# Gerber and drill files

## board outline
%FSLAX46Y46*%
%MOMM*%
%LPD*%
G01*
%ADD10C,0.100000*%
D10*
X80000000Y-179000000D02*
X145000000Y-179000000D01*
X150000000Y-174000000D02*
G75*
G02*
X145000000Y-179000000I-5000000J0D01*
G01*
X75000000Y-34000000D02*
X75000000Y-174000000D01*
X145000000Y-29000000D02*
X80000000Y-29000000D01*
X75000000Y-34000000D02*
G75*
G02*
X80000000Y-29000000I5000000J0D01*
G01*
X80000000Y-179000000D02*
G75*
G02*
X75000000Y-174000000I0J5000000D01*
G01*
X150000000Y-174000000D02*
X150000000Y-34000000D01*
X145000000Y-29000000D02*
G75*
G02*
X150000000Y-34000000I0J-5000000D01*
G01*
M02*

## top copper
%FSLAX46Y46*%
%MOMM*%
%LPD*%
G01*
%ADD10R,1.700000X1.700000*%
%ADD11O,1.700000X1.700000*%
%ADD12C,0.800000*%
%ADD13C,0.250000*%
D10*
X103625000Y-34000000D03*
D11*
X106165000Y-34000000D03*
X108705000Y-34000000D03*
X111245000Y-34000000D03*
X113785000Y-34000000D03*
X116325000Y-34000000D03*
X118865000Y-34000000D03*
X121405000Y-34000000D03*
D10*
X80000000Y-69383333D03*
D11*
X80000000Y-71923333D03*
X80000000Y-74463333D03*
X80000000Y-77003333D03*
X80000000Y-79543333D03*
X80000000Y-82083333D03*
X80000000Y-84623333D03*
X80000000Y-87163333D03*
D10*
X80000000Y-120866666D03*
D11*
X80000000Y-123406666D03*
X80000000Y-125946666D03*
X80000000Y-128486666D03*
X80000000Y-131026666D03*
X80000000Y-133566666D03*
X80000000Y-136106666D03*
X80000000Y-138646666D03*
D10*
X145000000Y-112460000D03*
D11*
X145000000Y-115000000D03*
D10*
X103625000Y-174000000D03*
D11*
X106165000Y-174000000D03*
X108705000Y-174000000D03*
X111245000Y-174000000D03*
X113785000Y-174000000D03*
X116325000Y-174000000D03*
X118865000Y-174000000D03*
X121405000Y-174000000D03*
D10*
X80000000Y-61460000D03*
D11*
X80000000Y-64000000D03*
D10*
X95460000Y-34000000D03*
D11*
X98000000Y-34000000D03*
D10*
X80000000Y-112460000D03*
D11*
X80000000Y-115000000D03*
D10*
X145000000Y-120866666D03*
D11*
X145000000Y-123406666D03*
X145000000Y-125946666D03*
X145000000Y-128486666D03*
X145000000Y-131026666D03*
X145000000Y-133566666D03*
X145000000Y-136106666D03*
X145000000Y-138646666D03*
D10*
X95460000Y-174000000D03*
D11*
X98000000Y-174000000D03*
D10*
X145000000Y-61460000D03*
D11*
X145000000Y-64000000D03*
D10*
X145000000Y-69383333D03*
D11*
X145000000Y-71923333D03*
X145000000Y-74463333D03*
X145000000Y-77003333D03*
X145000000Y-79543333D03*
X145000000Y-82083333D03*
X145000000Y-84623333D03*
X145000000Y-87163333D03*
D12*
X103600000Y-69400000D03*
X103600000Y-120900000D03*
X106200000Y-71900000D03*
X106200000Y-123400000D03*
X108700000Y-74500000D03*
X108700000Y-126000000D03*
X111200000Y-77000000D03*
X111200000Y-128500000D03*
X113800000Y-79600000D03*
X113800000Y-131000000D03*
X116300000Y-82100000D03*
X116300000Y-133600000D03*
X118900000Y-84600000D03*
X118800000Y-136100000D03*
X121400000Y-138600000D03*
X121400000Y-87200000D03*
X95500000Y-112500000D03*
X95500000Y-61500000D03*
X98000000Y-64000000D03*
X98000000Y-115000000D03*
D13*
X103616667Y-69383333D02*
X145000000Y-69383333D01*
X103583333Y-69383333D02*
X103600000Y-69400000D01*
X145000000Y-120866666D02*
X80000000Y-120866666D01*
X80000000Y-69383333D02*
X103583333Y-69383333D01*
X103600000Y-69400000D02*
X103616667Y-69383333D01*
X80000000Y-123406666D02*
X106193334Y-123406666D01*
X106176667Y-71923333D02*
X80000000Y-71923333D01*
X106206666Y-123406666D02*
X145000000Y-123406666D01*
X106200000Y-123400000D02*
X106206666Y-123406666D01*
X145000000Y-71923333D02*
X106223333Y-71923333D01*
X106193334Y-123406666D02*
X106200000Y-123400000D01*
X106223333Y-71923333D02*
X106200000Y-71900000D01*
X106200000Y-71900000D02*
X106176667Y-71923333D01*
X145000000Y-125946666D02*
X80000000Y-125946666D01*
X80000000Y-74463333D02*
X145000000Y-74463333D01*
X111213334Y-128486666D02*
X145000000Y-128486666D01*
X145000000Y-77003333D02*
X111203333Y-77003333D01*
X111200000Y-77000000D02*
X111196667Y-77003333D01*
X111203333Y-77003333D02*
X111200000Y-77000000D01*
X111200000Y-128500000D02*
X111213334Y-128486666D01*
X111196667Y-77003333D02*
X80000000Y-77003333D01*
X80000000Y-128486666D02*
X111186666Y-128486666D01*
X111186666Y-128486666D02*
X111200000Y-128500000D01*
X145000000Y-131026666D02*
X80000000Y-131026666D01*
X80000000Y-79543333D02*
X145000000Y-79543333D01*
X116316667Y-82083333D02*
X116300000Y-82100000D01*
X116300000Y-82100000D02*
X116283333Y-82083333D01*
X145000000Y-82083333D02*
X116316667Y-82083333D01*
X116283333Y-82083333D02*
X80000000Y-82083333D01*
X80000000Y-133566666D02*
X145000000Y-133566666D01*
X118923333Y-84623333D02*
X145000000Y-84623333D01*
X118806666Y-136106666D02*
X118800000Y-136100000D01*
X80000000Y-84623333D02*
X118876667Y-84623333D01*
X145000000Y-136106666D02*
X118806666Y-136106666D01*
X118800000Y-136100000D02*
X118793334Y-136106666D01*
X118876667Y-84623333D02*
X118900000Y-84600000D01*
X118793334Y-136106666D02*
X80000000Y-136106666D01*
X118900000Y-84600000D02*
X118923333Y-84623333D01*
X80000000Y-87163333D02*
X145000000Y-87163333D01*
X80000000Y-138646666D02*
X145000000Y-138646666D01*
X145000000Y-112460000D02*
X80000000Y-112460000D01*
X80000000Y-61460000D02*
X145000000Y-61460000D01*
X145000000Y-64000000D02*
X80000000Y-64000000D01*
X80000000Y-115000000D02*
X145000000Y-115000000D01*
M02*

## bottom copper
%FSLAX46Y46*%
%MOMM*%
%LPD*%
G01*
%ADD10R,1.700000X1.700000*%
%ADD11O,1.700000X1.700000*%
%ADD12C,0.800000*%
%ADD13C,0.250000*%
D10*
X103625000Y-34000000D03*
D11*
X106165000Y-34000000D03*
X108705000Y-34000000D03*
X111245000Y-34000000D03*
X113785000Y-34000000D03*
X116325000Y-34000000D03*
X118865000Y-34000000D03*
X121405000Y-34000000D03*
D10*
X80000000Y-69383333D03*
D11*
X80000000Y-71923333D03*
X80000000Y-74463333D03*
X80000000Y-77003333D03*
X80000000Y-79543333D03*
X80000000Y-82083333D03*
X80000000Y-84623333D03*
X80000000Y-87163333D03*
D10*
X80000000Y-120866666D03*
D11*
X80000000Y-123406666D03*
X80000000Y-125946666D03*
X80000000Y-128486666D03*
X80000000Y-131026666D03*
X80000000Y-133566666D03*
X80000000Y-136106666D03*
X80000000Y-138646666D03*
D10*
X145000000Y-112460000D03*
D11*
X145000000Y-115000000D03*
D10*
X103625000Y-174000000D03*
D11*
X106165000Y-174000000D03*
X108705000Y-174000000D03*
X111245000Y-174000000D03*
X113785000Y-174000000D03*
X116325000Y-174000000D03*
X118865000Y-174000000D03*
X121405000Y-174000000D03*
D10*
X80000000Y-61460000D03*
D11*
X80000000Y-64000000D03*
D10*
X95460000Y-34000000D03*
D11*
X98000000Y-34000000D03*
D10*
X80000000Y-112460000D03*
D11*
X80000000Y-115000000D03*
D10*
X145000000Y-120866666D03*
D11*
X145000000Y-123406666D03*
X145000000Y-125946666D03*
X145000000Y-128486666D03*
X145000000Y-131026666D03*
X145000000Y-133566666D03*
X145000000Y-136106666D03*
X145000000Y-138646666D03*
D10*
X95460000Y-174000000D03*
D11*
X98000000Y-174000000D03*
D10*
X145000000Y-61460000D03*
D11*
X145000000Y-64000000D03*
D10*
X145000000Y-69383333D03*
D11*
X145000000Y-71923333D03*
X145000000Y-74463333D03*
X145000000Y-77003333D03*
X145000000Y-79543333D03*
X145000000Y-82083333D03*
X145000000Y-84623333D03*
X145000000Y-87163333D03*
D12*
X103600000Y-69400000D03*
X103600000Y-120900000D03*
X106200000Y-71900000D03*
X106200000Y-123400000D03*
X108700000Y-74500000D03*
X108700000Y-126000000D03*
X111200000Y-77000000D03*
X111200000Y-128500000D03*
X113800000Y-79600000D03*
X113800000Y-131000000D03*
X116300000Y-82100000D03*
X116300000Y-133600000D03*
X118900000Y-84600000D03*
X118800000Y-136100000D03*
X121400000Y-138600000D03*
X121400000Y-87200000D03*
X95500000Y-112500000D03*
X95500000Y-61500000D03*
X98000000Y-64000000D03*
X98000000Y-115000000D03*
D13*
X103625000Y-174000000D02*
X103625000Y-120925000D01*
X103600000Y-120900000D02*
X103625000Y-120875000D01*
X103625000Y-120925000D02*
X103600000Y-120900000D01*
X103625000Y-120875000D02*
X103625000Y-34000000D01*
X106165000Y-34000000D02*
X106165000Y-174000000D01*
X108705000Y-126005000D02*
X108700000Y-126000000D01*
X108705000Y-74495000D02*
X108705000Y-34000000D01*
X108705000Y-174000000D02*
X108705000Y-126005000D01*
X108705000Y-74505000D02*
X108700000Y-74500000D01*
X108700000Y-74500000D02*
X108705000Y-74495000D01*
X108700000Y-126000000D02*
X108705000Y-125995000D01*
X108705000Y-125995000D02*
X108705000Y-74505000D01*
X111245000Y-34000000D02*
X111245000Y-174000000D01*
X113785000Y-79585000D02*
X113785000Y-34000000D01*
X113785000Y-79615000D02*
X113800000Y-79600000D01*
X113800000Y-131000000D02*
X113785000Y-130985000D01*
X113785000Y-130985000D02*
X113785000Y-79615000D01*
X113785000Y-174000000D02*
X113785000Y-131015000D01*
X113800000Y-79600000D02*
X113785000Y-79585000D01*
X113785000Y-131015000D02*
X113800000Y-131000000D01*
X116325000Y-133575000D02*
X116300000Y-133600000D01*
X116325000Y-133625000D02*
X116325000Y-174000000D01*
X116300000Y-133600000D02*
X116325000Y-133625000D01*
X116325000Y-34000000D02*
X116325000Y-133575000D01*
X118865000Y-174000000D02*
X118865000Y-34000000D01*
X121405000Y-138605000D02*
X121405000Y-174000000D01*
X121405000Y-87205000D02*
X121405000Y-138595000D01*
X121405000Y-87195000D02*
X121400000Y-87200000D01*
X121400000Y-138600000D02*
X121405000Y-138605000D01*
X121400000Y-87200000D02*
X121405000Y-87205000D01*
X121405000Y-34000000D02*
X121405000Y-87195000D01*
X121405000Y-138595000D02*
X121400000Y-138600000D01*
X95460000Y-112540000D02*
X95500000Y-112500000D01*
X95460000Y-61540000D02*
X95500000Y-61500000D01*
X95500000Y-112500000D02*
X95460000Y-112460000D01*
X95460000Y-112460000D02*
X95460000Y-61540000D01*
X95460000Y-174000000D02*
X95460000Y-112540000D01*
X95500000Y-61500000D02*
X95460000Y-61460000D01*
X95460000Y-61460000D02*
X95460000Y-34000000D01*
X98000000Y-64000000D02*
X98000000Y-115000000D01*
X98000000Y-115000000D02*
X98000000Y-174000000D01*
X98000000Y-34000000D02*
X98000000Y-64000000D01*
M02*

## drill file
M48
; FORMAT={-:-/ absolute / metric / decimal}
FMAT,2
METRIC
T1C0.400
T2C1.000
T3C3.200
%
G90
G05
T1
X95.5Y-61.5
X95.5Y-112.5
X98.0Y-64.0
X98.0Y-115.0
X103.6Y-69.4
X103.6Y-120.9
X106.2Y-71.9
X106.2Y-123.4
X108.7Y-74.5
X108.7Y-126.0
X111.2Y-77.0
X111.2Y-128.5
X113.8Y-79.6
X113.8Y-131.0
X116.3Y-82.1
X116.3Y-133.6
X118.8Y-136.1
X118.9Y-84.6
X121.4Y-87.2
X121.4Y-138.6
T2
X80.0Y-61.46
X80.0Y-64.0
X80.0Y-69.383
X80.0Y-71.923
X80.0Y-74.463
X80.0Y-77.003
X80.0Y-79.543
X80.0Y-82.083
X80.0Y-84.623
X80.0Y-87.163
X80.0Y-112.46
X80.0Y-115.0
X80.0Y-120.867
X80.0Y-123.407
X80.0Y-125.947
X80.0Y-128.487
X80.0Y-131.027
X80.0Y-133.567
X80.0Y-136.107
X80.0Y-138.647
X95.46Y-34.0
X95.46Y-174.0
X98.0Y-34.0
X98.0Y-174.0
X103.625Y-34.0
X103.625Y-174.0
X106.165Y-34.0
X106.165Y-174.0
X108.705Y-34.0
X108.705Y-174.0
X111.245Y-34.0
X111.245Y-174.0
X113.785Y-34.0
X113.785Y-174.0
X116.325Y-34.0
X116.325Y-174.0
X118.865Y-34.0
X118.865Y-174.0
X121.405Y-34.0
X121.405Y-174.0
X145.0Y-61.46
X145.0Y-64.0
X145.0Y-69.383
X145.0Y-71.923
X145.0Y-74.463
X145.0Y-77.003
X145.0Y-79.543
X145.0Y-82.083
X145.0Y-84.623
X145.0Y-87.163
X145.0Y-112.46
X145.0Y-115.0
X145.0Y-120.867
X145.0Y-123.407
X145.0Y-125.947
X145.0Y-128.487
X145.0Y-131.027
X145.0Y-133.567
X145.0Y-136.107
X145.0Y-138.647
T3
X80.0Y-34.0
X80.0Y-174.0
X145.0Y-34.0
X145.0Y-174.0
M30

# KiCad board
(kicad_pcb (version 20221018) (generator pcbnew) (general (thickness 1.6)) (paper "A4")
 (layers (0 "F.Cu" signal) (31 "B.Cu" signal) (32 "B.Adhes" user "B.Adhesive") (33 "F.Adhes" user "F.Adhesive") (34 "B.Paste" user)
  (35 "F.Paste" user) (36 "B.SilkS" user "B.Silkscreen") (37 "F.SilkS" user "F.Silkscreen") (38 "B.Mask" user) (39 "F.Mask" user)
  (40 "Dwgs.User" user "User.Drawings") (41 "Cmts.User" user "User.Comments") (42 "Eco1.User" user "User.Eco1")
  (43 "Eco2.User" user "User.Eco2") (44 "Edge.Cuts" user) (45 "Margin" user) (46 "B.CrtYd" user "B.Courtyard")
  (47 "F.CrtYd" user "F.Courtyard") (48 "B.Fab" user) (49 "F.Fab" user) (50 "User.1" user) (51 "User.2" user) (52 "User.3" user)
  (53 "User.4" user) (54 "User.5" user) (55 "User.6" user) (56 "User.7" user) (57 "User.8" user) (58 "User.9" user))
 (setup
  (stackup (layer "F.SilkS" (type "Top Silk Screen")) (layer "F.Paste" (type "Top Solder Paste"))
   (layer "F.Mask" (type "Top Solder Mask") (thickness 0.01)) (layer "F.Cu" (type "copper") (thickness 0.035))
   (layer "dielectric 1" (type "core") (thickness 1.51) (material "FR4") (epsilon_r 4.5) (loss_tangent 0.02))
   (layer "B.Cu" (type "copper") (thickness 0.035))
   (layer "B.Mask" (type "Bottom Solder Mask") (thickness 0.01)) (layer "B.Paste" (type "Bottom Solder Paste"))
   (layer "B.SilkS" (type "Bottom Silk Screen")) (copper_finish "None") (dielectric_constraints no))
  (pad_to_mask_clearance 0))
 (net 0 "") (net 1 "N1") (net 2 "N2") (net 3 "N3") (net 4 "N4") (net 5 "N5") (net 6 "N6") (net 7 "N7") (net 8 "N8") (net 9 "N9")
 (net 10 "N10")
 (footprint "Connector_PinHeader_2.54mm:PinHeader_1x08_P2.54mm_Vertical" (layer "F.Cu") (at 103.625 34 90)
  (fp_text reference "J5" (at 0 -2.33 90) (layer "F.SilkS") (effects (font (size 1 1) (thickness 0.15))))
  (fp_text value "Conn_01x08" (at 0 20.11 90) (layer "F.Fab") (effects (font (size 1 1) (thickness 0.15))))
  (pad "1" thru_hole rect (at 0 0 90) (size 1.7 1.7) (drill 1) (layers "*.Cu" "*.Mask") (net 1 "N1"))
  (pad "2" thru_hole oval (at 0 2.54 90) (size 1.7 1.7) (drill 1) (layers "*.Cu" "*.Mask") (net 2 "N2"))
  (pad "3" thru_hole oval (at 0 5.08 90) (size 1.7 1.7) (drill 1) (layers "*.Cu" "*.Mask") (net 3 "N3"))
  (pad "4" thru_hole oval (at 0 7.62 90) (size 1.7 1.7) (drill 1) (layers "*.Cu" "*.Mask") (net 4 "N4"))
  (pad "5" thru_hole oval (at 0 10.16 90) (size 1.7 1.7) (drill 1) (layers "*.Cu" "*.Mask") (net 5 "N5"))
  (pad "6" thru_hole oval (at 0 12.7 90) (size 1.7 1.7) (drill 1) (layers "*.Cu" "*.Mask") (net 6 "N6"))
  (pad "7" thru_hole oval (at 0 15.24 90) (size 1.7 1.7) (drill 1) (layers "*.Cu" "*.Mask") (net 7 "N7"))
  (pad "8" thru_hole oval (at 0 17.78 90) (size 1.7 1.7) (drill 1) (layers "*.Cu" "*.Mask") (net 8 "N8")))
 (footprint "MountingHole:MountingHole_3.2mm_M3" (layer "F.Cu") (at 80 174)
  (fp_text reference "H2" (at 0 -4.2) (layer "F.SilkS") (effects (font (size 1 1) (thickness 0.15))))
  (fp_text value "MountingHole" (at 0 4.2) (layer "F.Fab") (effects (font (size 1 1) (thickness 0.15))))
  (pad "" np_thru_hole circle (at 0 0) (size 3.2 3.2) (drill 3.2) (layers "*.Cu" "*.Mask")))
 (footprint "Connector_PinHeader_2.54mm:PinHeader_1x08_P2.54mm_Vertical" (layer "F.Cu") (at 80 69.383333)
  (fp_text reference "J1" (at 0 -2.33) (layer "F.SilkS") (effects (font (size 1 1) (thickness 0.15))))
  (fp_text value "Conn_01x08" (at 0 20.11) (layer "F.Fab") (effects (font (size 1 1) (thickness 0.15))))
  (pad "1" thru_hole rect (at 0 0) (size 1.7 1.7) (drill 1) (layers "*.Cu" "*.Mask") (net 1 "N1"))
  (pad "2" thru_hole oval (at 0 2.54) (size 1.7 1.7) (drill 1) (layers "*.Cu" "*.Mask") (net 2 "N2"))
  (pad "3" thru_hole oval (at 0 5.08) (size 1.7 1.7) (drill 1) (layers "*.Cu" "*.Mask") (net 3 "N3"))
  (pad "4" thru_hole oval (at 0 7.62) (size 1.7 1.7) (drill 1) (layers "*.Cu" "*.Mask") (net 4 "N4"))
  (pad "5" thru_hole oval (at 0 10.16) (size 1.7 1.7) (drill 1) (layers "*.Cu" "*.Mask") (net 5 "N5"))
  (pad "6" thru_hole oval (at 0 12.7) (size 1.7 1.7) (drill 1) (layers "*.Cu" "*.Mask") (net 6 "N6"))
  (pad "7" thru_hole oval (at 0 15.24) (size 1.7 1.7) (drill 1) (layers "*.Cu" "*.Mask") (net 7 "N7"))
  (pad "8" thru_hole oval (at 0 17.78) (size 1.7 1.7) (drill 1) (layers "*.Cu" "*.Mask") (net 8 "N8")))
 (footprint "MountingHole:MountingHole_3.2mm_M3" (layer "F.Cu") (at 145 174)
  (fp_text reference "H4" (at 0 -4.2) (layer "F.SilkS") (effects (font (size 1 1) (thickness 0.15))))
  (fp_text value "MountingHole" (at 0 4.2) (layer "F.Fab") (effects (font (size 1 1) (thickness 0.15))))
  (pad "" np_thru_hole circle (at 0 0) (size 3.2 3.2) (drill 3.2) (layers "*.Cu" "*.Mask")))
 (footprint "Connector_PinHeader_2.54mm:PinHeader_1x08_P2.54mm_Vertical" (layer "F.Cu") (at 80 120.866666)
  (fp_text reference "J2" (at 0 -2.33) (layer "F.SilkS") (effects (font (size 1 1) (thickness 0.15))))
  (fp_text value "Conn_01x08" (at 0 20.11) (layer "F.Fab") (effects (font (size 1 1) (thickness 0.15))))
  (pad "1" thru_hole rect (at 0 0) (size 1.7 1.7) (drill 1) (layers "*.Cu" "*.Mask") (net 1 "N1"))
  (pad "2" thru_hole oval (at 0 2.54) (size 1.7 1.7) (drill 1) (layers "*.Cu" "*.Mask") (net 2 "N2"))
  (pad "3" thru_hole oval (at 0 5.08) (size 1.7 1.7) (drill 1) (layers "*.Cu" "*.Mask") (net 3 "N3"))
  (pad "4" thru_hole oval (at 0 7.62) (size 1.7 1.7) (drill 1) (layers "*.Cu" "*.Mask") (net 4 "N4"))
  (pad "5" thru_hole oval (at 0 10.16) (size 1.7 1.7) (drill 1) (layers "*.Cu" "*.Mask") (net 5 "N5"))
  (pad "6" thru_hole oval (at 0 12.7) (size 1.7 1.7) (drill 1) (layers "*.Cu" "*.Mask") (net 6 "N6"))
  (pad "7" thru_hole oval (at 0 15.24) (size 1.7 1.7) (drill 1) (layers "*.Cu" "*.Mask") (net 7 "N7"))
  (pad "8" thru_hole oval (at 0 17.78) (size 1.7 1.7) (drill 1) (layers "*.Cu" "*.Mask") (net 8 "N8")))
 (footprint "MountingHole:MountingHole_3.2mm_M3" (layer "F.Cu") (at 80 34)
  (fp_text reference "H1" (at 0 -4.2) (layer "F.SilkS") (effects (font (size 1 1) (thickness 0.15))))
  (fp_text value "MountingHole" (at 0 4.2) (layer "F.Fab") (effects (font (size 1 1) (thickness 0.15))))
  (pad "" np_thru_hole circle (at 0 0) (size 3.2 3.2) (drill 3.2) (layers "*.Cu" "*.Mask")))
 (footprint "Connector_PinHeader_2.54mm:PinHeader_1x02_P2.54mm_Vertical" (layer "F.Cu") (at 145 112.46)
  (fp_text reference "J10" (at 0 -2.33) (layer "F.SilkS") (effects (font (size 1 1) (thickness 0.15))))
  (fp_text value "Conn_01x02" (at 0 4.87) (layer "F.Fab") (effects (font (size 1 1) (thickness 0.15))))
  (pad "1" thru_hole rect (at 0 0) (size 1.7 1.7) (drill 1) (layers "*.Cu" "*.Mask") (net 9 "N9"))
  (pad "2" thru_hole oval (at 0 2.54) (size 1.7 1.7) (drill 1) (layers "*.Cu" "*.Mask") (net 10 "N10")))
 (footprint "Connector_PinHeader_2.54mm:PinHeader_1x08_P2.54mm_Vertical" (layer "F.Cu") (at 103.625 174 90)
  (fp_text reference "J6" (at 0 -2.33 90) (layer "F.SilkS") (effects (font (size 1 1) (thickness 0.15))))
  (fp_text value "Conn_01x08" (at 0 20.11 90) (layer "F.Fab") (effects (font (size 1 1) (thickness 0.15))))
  (pad "1" thru_hole rect (at 0 0 90) (size 1.7 1.7) (drill 1) (layers "*.Cu" "*.Mask") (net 1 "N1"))
  (pad "2" thru_hole oval (at 0 2.54 90) (size 1.7 1.7) (drill 1) (layers "*.Cu" "*.Mask") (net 2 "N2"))
  (pad "3" thru_hole oval (at 0 5.08 90) (size 1.7 1.7) (drill 1) (layers "*.Cu" "*.Mask") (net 3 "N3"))
  (pad "4" thru_hole oval (at 0 7.62 90) (size 1.7 1.7) (drill 1) (layers "*.Cu" "*.Mask") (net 4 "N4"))
  (pad "5" thru_hole oval (at 0 10.16 90) (size 1.7 1.7) (drill 1) (layers "*.Cu" "*.Mask") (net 5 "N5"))
  (pad "6" thru_hole oval (at 0 12.7 90) (size 1.7 1.7) (drill 1) (layers "*.Cu" "*.Mask") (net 6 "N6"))
  (pad "7" thru_hole oval (at 0 15.24 90) (size 1.7 1.7) (drill 1) (layers "*.Cu" "*.Mask") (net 7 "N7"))
  (pad "8" thru_hole oval (at 0 17.78 90) (size 1.7 1.7) (drill 1) (layers "*.Cu" "*.Mask") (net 8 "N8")))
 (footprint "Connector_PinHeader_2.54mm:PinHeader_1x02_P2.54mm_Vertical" (layer "F.Cu") (at 80 61.46)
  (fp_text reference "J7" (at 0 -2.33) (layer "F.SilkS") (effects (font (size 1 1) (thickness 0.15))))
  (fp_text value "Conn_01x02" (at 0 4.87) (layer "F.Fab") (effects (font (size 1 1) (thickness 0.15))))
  (pad "1" thru_hole rect (at 0 0) (size 1.7 1.7) (drill 1) (layers "*.Cu" "*.Mask") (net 9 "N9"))
  (pad "2" thru_hole oval (at 0 2.54) (size 1.7 1.7) (drill 1) (layers "*.Cu" "*.Mask") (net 10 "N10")))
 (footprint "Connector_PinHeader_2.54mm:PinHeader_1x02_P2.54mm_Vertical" (layer "F.Cu") (at 95.46 34 90)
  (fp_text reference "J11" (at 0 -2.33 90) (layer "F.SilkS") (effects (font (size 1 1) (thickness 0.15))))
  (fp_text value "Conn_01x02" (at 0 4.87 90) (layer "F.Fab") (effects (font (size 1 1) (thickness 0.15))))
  (pad "1" thru_hole rect (at 0 0 90) (size 1.7 1.7) (drill 1) (layers "*.Cu" "*.Mask") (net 9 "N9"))
  (pad "2" thru_hole oval (at 0 2.54 90) (size 1.7 1.7) (drill 1) (layers "*.Cu" "*.Mask") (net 10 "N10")))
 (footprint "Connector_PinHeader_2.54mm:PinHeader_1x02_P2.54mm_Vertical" (layer "F.Cu") (at 80 112.46)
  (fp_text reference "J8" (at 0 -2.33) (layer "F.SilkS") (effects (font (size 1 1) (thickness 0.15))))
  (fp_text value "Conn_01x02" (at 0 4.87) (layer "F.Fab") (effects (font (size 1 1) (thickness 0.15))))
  (pad "1" thru_hole rect (at 0 0) (size 1.7 1.7) (drill 1) (layers "*.Cu" "*.Mask") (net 9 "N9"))
  (pad "2" thru_hole oval (at 0 2.54) (size 1.7 1.7) (drill 1) (layers "*.Cu" "*.Mask") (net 10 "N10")))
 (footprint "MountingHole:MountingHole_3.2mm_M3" (layer "F.Cu") (at 145 34)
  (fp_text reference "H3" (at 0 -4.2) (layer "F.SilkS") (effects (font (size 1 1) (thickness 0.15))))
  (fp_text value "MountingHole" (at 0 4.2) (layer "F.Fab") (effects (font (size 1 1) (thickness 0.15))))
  (pad "" np_thru_hole circle (at 0 0) (size 3.2 3.2) (drill 3.2) (layers "*.Cu" "*.Mask")))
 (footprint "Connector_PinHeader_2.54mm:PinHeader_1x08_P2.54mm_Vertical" (layer "F.Cu") (at 145 120.866666)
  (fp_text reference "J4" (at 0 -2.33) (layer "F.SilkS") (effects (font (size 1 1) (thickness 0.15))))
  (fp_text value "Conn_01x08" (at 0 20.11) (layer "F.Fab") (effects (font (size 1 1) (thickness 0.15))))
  (pad "1" thru_hole rect (at 0 0) (size 1.7 1.7) (drill 1) (layers "*.Cu" "*.Mask") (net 1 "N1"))
  (pad "2" thru_hole oval (at 0 2.54) (size 1.7 1.7) (drill 1) (layers "*.Cu" "*.Mask") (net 2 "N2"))
  (pad "3" thru_hole oval (at 0 5.08) (size 1.7 1.7) (drill 1) (layers "*.Cu" "*.Mask") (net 3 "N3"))
  (pad "4" thru_hole oval (at 0 7.62) (size 1.7 1.7) (drill 1) (layers "*.Cu" "*.Mask") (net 4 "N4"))
  (pad "5" thru_hole oval (at 0 10.16) (size 1.7 1.7) (drill 1) (layers "*.Cu" "*.Mask") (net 5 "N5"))
  (pad "6" thru_hole oval (at 0 12.7) (size 1.7 1.7) (drill 1) (layers "*.Cu" "*.Mask") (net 6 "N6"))
  (pad "7" thru_hole oval (at 0 15.24) (size 1.7 1.7) (drill 1) (layers "*.Cu" "*.Mask") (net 7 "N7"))
  (pad "8" thru_hole oval (at 0 17.78) (size 1.7 1.7) (drill 1) (layers "*.Cu" "*.Mask") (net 8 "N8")))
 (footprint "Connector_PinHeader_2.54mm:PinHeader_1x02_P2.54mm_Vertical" (layer "F.Cu") (at 95.46 174 90)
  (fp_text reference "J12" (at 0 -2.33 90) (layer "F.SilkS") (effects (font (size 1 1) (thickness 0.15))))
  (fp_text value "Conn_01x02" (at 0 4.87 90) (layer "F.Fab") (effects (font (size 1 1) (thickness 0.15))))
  (pad "1" thru_hole rect (at 0 0 90) (size 1.7 1.7) (drill 1) (layers "*.Cu" "*.Mask") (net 9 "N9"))
  (pad "2" thru_hole oval (at 0 2.54 90) (size 1.7 1.7) (drill 1) (layers "*.Cu" "*.Mask") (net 10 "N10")))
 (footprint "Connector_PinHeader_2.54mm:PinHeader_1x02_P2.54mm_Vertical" (layer "F.Cu") (at 145 61.46)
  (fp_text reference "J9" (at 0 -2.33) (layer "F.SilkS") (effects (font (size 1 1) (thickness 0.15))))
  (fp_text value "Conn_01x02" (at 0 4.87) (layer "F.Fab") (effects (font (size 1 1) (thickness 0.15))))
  (pad "1" thru_hole rect (at 0 0) (size 1.7 1.7) (drill 1) (layers "*.Cu" "*.Mask") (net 9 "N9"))
  (pad "2" thru_hole oval (at 0 2.54) (size 1.7 1.7) (drill 1) (layers "*.Cu" "*.Mask") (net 10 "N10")))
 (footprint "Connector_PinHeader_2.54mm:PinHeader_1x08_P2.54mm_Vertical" (layer "F.Cu") (at 145 69.383333)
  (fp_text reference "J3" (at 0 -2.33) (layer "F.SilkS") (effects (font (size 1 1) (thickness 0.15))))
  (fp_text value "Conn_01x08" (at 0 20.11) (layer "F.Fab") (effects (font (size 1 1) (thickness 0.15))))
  (pad "1" thru_hole rect (at 0 0) (size 1.7 1.7) (drill 1) (layers "*.Cu" "*.Mask") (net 1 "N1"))
  (pad "2" thru_hole oval (at 0 2.54) (size 1.7 1.7) (drill 1) (layers "*.Cu" "*.Mask") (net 2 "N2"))
  (pad "3" thru_hole oval (at 0 5.08) (size 1.7 1.7) (drill 1) (layers "*.Cu" "*.Mask") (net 3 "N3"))
  (pad "4" thru_hole oval (at 0 7.62) (size 1.7 1.7) (drill 1) (layers "*.Cu" "*.Mask") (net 4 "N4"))
  (pad "5" thru_hole oval (at 0 10.16) (size 1.7 1.7) (drill 1) (layers "*.Cu" "*.Mask") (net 5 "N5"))
  (pad "6" thru_hole oval (at 0 12.7) (size 1.7 1.7) (drill 1) (layers "*.Cu" "*.Mask") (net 6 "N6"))
  (pad "7" thru_hole oval (at 0 15.24) (size 1.7 1.7) (drill 1) (layers "*.Cu" "*.Mask") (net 7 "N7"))
  (pad "8" thru_hole oval (at 0 17.78) (size 1.7 1.7) (drill 1) (layers "*.Cu" "*.Mask") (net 8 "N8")))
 (gr_line (start 80 179) (end 145 179) (stroke (width 0.1) (type default)) (layer "Edge.Cuts"))
 (gr_arc (start 150 174) (mid 148.535534 177.535534) (end 145 179) (stroke (width 0.1) (type default)) (layer "Edge.Cuts"))
 (gr_line (start 75 34) (end 75 174) (stroke (width 0.1) (type default)) (layer "Edge.Cuts"))
 (gr_line (start 145 29) (end 80 29) (stroke (width 0.1) (type default)) (layer "Edge.Cuts"))
 (gr_arc (start 75 34) (mid 76.464466 30.464466) (end 80 29) (stroke (width 0.1) (type default)) (layer "Edge.Cuts"))
 (gr_arc (start 80 179) (mid 76.464466 177.535534) (end 75 174) (stroke (width 0.1) (type default)) (layer "Edge.Cuts"))
 (gr_line (start 150 174) (end 150 34) (stroke (width 0.1) (type default)) (layer "Edge.Cuts"))
 (gr_arc (start 145 29) (mid 148.535534 30.464466) (end 150 34) (stroke (width 0.1) (type default)) (layer "Edge.Cuts"))
 (segment (start 103.616667 69.383333) (end 145 69.383333) (width 0.25) (layer "F.Cu") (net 1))
 (segment (start 103.583333 69.383333) (end 103.6 69.4) (width 0.25) (layer "F.Cu") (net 1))
 (segment (start 145 120.866666) (end 80 120.866666) (width 0.25) (layer "F.Cu") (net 1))
 (segment (start 80 69.383333) (end 103.583333 69.383333) (width 0.25) (layer "F.Cu") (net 1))
 (segment (start 103.6 69.4) (end 103.616667 69.383333) (width 0.25) (layer "F.Cu") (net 1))
 (via (at 103.6 69.4) (size 0.8) (drill 0.4) (layers "F.Cu" "B.Cu") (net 1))
 (via (at 103.6 120.9) (size 0.8) (drill 0.4) (layers "F.Cu" "B.Cu") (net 1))
 (segment (start 103.625 174) (end 103.625 120.925) (width 0.25) (layer "B.Cu") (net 1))
 (segment (start 103.6 120.9) (end 103.625 120.875) (width 0.25) (layer "B.Cu") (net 1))
 (segment (start 103.625 120.925) (end 103.6 120.9) (width 0.25) (layer "B.Cu") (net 1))
 (segment (start 103.625 120.875) (end 103.625 34) (width 0.25) (layer "B.Cu") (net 1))
 (segment (start 80 123.406666) (end 106.193334 123.406666) (width 0.25) (layer "F.Cu") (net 2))
 (segment (start 106.176667 71.923333) (end 80 71.923333) (width 0.25) (layer "F.Cu") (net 2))
 (segment (start 106.206666 123.406666) (end 145 123.406666) (width 0.25) (layer "F.Cu") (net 2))
 (segment (start 106.2 123.4) (end 106.206666 123.406666) (width 0.25) (layer "F.Cu") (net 2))
 (segment (start 145 71.923333) (end 106.223333 71.923333) (width 0.25) (layer "F.Cu") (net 2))
 (segment (start 106.193334 123.406666) (end 106.2 123.4) (width 0.25) (layer "F.Cu") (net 2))
 (segment (start 106.223333 71.923333) (end 106.2 71.9) (width 0.25) (layer "F.Cu") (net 2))
 (segment (start 106.2 71.9) (end 106.176667 71.923333) (width 0.25) (layer "F.Cu") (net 2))
 (via (at 106.2 71.9) (size 0.8) (drill 0.4) (layers "F.Cu" "B.Cu") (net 2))
 (via (at 106.2 123.4) (size 0.8) (drill 0.4) (layers "F.Cu" "B.Cu") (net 2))
 (segment (start 106.165 34) (end 106.165 174) (width 0.25) (layer "B.Cu") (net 2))
 (segment (start 145 125.946666) (end 80 125.946666) (width 0.25) (layer "F.Cu") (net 3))
 (segment (start 80 74.463333) (end 145 74.463333) (width 0.25) (layer "F.Cu") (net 3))
 (via (at 108.7 74.5) (size 0.8) (drill 0.4) (layers "F.Cu" "B.Cu") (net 3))
 (via (at 108.7 126) (size 0.8) (drill 0.4) (layers "F.Cu" "B.Cu") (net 3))
 (segment (start 108.705 126.005) (end 108.7 126) (width 0.25) (layer "B.Cu") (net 3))
 (segment (start 108.705 74.495) (end 108.705 34) (width 0.25) (layer "B.Cu") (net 3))
 (segment (start 108.705 174) (end 108.705 126.005) (width 0.25) (layer "B.Cu") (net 3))
 (segment (start 108.705 74.505) (end 108.7 74.5) (width 0.25) (layer "B.Cu") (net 3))
 (segment (start 108.7 74.5) (end 108.705 74.495) (width 0.25) (layer "B.Cu") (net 3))
 (segment (start 108.7 126) (end 108.705 125.995) (width 0.25) (layer "B.Cu") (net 3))
 (segment (start 108.705 125.995) (end 108.705 74.505) (width 0.25) (layer "B.Cu") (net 3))
 (segment (start 111.213334 128.486666) (end 145 128.486666) (width 0.25) (layer "F.Cu") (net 4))
 (segment (start 145 77.003333) (end 111.203333 77.003333) (width 0.25) (layer "F.Cu") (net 4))
 (segment (start 111.2 77) (end 111.196667 77.003333) (width 0.25) (layer "F.Cu") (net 4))
 (segment (start 111.203333 77.003333) (end 111.2 77) (width 0.25) (layer "F.Cu") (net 4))
 (segment (start 111.2 128.5) (end 111.213334 128.486666) (width 0.25) (layer "F.Cu") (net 4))
 (segment (start 111.196667 77.003333) (end 80 77.003333) (width 0.25) (layer "F.Cu") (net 4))
 (segment (start 80 128.486666) (end 111.186666 128.486666) (width 0.25) (layer "F.Cu") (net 4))
 (segment (start 111.186666 128.486666) (end 111.2 128.5) (width 0.25) (layer "F.Cu") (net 4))
 (via (at 111.2 77) (size 0.8) (drill 0.4) (layers "F.Cu" "B.Cu") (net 4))
 (via (at 111.2 128.5) (size 0.8) (drill 0.4) (layers "F.Cu" "B.Cu") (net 4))
 (segment (start 111.245 34) (end 111.245 174) (width 0.25) (layer "B.Cu") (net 4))
 (segment (start 145 131.026666) (end 80 131.026666) (width 0.25) (layer "F.Cu") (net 5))
 (segment (start 80 79.543333) (end 145 79.543333) (width 0.25) (layer "F.Cu") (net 5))
 (via (at 113.8 79.6) (size 0.8) (drill 0.4) (layers "F.Cu" "B.Cu") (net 5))
 (via (at 113.8 131) (size 0.8) (drill 0.4) (layers "F.Cu" "B.Cu") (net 5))
 (segment (start 113.785 79.585) (end 113.785 34) (width 0.25) (layer "B.Cu") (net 5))
 (segment (start 113.785 79.615) (end 113.8 79.6) (width 0.25) (layer "B.Cu") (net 5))
 (segment (start 113.8 131) (end 113.785 130.985) (width 0.25) (layer "B.Cu") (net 5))
 (segment (start 113.785 130.985) (end 113.785 79.615) (width 0.25) (layer "B.Cu") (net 5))
 (segment (start 113.785 174) (end 113.785 131.015) (width 0.25) (layer "B.Cu") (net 5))
 (segment (start 113.8 79.6) (end 113.785 79.585) (width 0.25) (layer "B.Cu") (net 5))
 (segment (start 113.785 131.015) (end 113.8 131) (width 0.25) (layer "B.Cu") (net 5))
 (segment (start 116.316667 82.083333) (end 116.3 82.1) (width 0.25) (layer "F.Cu") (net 6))
 (segment (start 116.3 82.1) (end 116.283333 82.083333) (width 0.25) (layer "F.Cu") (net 6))
 (segment (start 145 82.083333) (end 116.316667 82.083333) (width 0.25) (layer "F.Cu") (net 6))
 (segment (start 116.283333 82.083333) (end 80 82.083333) (width 0.25) (layer "F.Cu") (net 6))
 (segment (start 80 133.566666) (end 145 133.566666) (width 0.25) (layer "F.Cu") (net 6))
 (via (at 116.3 82.1) (size 0.8) (drill 0.4) (layers "F.Cu" "B.Cu") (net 6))
 (via (at 116.3 133.6) (size 0.8) (drill 0.4) (layers "F.Cu" "B.Cu") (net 6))
 (segment (start 116.325 133.575) (end 116.3 133.6) (width 0.25) (layer "B.Cu") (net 6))
 (segment (start 116.325 133.625) (end 116.325 174) (width 0.25) (layer "B.Cu") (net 6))
 (segment (start 116.3 133.6) (end 116.325 133.625) (width 0.25) (layer "B.Cu") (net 6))
 (segment (start 116.325 34) (end 116.325 133.575) (width 0.25) (layer "B.Cu") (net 6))
 (segment (start 118.923333 84.623333) (end 145 84.623333) (width 0.25) (layer "F.Cu") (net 7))
 (segment (start 118.806666 136.106666) (end 118.8 136.1) (width 0.25) (layer "F.Cu") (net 7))
 (segment (start 80 84.623333) (end 118.876667 84.623333) (width 0.25) (layer "F.Cu") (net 7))
 (segment (start 145 136.106666) (end 118.806666 136.106666) (width 0.25) (layer "F.Cu") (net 7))
 (segment (start 118.8 136.1) (end 118.793334 136.106666) (width 0.25) (layer "F.Cu") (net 7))
 (segment (start 118.876667 84.623333) (end 118.9 84.6) (width 0.25) (layer "F.Cu") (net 7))
 (segment (start 118.793334 136.106666) (end 80 136.106666) (width 0.25) (layer "F.Cu") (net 7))
 (segment (start 118.9 84.6) (end 118.923333 84.623333) (width 0.25) (layer "F.Cu") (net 7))
 (via (at 118.9 84.6) (size 0.8) (drill 0.4) (layers "F.Cu" "B.Cu") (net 7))
 (via (at 118.8 136.1) (size 0.8) (drill 0.4) (layers "F.Cu" "B.Cu") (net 7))
 (segment (start 118.865 174) (end 118.865 34) (width 0.25) (layer "B.Cu") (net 7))
 (segment (start 80 87.163333) (end 145 87.163333) (width 0.25) (layer "F.Cu") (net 8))
 (segment (start 80 138.646666) (end 145 138.646666) (width 0.25) (layer "F.Cu") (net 8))
 (via (at 121.4 138.6) (size 0.8) (drill 0.4) (layers "F.Cu" "B.Cu") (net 8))
 (via (at 121.4 87.2) (size 0.8) (drill 0.4) (layers "F.Cu" "B.Cu") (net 8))
 (segment (start 121.405 138.605) (end 121.405 174) (width 0.25) (layer "B.Cu") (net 8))
 (segment (start 121.405 87.205) (end 121.405 138.595) (width 0.25) (layer "B.Cu") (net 8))
 (segment (start 121.405 87.195) (end 121.4 87.2) (width 0.25) (layer "B.Cu") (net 8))
 (segment (start 121.4 138.6) (end 121.405 138.605) (width 0.25) (layer "B.Cu") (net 8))
 (segment (start 121.4 87.2) (end 121.405 87.205) (width 0.25) (layer "B.Cu") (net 8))
 (segment (start 121.405 34) (end 121.405 87.195) (width 0.25) (layer "B.Cu") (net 8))
 (segment (start 121.405 138.595) (end 121.4 138.6) (width 0.25) (layer "B.Cu") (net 8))
 (segment (start 145 112.46) (end 80 112.46) (width 0.25) (layer "F.Cu") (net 9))
 (segment (start 80 61.46) (end 145 61.46) (width 0.25) (layer "F.Cu") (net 9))
 (via (at 95.5 112.5) (size 0.8) (drill 0.4) (layers "F.Cu" "B.Cu") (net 9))
 (via (at 95.5 61.5) (size 0.8) (drill 0.4) (layers "F.Cu" "B.Cu") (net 9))
 (segment (start 95.46 112.54) (end 95.5 112.5) (width 0.25) (layer "B.Cu") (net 9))
 (segment (start 95.46 61.54) (end 95.5 61.5) (width 0.25) (layer "B.Cu") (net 9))
 (segment (start 95.5 112.5) (end 95.46 112.46) (width 0.25) (layer "B.Cu") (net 9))
 (segment (start 95.46 112.46) (end 95.46 61.54) (width 0.25) (layer "B.Cu") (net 9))
 (segment (start 95.46 174) (end 95.46 112.54) (width 0.25) (layer "B.Cu") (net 9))
 (segment (start 95.5 61.5) (end 95.46 61.46) (width 0.25) (layer "B.Cu") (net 9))
 (segment (start 95.46 61.46) (end 95.46 34) (width 0.25) (layer "B.Cu") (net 9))
 (segment (start 145 64) (end 80 64) (width 0.25) (layer "F.Cu") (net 10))
 (segment (start 80 115) (end 145 115) (width 0.25) (layer "F.Cu") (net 10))
 (via (at 98 64) (size 0.8) (drill 0.4) (layers "F.Cu" "B.Cu") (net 10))
 (via (at 98 115) (size 0.8) (drill 0.4) (layers "F.Cu" "B.Cu") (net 10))
 (segment (start 98 64) (end 98 115) (width 0.25) (layer "B.Cu") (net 10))
 (segment (start 98 115) (end 98 174) (width 0.25) (layer "B.Cu") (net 10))
 (segment (start 98 34) (end 98 64) (width 0.25) (layer "B.Cu") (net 10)))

